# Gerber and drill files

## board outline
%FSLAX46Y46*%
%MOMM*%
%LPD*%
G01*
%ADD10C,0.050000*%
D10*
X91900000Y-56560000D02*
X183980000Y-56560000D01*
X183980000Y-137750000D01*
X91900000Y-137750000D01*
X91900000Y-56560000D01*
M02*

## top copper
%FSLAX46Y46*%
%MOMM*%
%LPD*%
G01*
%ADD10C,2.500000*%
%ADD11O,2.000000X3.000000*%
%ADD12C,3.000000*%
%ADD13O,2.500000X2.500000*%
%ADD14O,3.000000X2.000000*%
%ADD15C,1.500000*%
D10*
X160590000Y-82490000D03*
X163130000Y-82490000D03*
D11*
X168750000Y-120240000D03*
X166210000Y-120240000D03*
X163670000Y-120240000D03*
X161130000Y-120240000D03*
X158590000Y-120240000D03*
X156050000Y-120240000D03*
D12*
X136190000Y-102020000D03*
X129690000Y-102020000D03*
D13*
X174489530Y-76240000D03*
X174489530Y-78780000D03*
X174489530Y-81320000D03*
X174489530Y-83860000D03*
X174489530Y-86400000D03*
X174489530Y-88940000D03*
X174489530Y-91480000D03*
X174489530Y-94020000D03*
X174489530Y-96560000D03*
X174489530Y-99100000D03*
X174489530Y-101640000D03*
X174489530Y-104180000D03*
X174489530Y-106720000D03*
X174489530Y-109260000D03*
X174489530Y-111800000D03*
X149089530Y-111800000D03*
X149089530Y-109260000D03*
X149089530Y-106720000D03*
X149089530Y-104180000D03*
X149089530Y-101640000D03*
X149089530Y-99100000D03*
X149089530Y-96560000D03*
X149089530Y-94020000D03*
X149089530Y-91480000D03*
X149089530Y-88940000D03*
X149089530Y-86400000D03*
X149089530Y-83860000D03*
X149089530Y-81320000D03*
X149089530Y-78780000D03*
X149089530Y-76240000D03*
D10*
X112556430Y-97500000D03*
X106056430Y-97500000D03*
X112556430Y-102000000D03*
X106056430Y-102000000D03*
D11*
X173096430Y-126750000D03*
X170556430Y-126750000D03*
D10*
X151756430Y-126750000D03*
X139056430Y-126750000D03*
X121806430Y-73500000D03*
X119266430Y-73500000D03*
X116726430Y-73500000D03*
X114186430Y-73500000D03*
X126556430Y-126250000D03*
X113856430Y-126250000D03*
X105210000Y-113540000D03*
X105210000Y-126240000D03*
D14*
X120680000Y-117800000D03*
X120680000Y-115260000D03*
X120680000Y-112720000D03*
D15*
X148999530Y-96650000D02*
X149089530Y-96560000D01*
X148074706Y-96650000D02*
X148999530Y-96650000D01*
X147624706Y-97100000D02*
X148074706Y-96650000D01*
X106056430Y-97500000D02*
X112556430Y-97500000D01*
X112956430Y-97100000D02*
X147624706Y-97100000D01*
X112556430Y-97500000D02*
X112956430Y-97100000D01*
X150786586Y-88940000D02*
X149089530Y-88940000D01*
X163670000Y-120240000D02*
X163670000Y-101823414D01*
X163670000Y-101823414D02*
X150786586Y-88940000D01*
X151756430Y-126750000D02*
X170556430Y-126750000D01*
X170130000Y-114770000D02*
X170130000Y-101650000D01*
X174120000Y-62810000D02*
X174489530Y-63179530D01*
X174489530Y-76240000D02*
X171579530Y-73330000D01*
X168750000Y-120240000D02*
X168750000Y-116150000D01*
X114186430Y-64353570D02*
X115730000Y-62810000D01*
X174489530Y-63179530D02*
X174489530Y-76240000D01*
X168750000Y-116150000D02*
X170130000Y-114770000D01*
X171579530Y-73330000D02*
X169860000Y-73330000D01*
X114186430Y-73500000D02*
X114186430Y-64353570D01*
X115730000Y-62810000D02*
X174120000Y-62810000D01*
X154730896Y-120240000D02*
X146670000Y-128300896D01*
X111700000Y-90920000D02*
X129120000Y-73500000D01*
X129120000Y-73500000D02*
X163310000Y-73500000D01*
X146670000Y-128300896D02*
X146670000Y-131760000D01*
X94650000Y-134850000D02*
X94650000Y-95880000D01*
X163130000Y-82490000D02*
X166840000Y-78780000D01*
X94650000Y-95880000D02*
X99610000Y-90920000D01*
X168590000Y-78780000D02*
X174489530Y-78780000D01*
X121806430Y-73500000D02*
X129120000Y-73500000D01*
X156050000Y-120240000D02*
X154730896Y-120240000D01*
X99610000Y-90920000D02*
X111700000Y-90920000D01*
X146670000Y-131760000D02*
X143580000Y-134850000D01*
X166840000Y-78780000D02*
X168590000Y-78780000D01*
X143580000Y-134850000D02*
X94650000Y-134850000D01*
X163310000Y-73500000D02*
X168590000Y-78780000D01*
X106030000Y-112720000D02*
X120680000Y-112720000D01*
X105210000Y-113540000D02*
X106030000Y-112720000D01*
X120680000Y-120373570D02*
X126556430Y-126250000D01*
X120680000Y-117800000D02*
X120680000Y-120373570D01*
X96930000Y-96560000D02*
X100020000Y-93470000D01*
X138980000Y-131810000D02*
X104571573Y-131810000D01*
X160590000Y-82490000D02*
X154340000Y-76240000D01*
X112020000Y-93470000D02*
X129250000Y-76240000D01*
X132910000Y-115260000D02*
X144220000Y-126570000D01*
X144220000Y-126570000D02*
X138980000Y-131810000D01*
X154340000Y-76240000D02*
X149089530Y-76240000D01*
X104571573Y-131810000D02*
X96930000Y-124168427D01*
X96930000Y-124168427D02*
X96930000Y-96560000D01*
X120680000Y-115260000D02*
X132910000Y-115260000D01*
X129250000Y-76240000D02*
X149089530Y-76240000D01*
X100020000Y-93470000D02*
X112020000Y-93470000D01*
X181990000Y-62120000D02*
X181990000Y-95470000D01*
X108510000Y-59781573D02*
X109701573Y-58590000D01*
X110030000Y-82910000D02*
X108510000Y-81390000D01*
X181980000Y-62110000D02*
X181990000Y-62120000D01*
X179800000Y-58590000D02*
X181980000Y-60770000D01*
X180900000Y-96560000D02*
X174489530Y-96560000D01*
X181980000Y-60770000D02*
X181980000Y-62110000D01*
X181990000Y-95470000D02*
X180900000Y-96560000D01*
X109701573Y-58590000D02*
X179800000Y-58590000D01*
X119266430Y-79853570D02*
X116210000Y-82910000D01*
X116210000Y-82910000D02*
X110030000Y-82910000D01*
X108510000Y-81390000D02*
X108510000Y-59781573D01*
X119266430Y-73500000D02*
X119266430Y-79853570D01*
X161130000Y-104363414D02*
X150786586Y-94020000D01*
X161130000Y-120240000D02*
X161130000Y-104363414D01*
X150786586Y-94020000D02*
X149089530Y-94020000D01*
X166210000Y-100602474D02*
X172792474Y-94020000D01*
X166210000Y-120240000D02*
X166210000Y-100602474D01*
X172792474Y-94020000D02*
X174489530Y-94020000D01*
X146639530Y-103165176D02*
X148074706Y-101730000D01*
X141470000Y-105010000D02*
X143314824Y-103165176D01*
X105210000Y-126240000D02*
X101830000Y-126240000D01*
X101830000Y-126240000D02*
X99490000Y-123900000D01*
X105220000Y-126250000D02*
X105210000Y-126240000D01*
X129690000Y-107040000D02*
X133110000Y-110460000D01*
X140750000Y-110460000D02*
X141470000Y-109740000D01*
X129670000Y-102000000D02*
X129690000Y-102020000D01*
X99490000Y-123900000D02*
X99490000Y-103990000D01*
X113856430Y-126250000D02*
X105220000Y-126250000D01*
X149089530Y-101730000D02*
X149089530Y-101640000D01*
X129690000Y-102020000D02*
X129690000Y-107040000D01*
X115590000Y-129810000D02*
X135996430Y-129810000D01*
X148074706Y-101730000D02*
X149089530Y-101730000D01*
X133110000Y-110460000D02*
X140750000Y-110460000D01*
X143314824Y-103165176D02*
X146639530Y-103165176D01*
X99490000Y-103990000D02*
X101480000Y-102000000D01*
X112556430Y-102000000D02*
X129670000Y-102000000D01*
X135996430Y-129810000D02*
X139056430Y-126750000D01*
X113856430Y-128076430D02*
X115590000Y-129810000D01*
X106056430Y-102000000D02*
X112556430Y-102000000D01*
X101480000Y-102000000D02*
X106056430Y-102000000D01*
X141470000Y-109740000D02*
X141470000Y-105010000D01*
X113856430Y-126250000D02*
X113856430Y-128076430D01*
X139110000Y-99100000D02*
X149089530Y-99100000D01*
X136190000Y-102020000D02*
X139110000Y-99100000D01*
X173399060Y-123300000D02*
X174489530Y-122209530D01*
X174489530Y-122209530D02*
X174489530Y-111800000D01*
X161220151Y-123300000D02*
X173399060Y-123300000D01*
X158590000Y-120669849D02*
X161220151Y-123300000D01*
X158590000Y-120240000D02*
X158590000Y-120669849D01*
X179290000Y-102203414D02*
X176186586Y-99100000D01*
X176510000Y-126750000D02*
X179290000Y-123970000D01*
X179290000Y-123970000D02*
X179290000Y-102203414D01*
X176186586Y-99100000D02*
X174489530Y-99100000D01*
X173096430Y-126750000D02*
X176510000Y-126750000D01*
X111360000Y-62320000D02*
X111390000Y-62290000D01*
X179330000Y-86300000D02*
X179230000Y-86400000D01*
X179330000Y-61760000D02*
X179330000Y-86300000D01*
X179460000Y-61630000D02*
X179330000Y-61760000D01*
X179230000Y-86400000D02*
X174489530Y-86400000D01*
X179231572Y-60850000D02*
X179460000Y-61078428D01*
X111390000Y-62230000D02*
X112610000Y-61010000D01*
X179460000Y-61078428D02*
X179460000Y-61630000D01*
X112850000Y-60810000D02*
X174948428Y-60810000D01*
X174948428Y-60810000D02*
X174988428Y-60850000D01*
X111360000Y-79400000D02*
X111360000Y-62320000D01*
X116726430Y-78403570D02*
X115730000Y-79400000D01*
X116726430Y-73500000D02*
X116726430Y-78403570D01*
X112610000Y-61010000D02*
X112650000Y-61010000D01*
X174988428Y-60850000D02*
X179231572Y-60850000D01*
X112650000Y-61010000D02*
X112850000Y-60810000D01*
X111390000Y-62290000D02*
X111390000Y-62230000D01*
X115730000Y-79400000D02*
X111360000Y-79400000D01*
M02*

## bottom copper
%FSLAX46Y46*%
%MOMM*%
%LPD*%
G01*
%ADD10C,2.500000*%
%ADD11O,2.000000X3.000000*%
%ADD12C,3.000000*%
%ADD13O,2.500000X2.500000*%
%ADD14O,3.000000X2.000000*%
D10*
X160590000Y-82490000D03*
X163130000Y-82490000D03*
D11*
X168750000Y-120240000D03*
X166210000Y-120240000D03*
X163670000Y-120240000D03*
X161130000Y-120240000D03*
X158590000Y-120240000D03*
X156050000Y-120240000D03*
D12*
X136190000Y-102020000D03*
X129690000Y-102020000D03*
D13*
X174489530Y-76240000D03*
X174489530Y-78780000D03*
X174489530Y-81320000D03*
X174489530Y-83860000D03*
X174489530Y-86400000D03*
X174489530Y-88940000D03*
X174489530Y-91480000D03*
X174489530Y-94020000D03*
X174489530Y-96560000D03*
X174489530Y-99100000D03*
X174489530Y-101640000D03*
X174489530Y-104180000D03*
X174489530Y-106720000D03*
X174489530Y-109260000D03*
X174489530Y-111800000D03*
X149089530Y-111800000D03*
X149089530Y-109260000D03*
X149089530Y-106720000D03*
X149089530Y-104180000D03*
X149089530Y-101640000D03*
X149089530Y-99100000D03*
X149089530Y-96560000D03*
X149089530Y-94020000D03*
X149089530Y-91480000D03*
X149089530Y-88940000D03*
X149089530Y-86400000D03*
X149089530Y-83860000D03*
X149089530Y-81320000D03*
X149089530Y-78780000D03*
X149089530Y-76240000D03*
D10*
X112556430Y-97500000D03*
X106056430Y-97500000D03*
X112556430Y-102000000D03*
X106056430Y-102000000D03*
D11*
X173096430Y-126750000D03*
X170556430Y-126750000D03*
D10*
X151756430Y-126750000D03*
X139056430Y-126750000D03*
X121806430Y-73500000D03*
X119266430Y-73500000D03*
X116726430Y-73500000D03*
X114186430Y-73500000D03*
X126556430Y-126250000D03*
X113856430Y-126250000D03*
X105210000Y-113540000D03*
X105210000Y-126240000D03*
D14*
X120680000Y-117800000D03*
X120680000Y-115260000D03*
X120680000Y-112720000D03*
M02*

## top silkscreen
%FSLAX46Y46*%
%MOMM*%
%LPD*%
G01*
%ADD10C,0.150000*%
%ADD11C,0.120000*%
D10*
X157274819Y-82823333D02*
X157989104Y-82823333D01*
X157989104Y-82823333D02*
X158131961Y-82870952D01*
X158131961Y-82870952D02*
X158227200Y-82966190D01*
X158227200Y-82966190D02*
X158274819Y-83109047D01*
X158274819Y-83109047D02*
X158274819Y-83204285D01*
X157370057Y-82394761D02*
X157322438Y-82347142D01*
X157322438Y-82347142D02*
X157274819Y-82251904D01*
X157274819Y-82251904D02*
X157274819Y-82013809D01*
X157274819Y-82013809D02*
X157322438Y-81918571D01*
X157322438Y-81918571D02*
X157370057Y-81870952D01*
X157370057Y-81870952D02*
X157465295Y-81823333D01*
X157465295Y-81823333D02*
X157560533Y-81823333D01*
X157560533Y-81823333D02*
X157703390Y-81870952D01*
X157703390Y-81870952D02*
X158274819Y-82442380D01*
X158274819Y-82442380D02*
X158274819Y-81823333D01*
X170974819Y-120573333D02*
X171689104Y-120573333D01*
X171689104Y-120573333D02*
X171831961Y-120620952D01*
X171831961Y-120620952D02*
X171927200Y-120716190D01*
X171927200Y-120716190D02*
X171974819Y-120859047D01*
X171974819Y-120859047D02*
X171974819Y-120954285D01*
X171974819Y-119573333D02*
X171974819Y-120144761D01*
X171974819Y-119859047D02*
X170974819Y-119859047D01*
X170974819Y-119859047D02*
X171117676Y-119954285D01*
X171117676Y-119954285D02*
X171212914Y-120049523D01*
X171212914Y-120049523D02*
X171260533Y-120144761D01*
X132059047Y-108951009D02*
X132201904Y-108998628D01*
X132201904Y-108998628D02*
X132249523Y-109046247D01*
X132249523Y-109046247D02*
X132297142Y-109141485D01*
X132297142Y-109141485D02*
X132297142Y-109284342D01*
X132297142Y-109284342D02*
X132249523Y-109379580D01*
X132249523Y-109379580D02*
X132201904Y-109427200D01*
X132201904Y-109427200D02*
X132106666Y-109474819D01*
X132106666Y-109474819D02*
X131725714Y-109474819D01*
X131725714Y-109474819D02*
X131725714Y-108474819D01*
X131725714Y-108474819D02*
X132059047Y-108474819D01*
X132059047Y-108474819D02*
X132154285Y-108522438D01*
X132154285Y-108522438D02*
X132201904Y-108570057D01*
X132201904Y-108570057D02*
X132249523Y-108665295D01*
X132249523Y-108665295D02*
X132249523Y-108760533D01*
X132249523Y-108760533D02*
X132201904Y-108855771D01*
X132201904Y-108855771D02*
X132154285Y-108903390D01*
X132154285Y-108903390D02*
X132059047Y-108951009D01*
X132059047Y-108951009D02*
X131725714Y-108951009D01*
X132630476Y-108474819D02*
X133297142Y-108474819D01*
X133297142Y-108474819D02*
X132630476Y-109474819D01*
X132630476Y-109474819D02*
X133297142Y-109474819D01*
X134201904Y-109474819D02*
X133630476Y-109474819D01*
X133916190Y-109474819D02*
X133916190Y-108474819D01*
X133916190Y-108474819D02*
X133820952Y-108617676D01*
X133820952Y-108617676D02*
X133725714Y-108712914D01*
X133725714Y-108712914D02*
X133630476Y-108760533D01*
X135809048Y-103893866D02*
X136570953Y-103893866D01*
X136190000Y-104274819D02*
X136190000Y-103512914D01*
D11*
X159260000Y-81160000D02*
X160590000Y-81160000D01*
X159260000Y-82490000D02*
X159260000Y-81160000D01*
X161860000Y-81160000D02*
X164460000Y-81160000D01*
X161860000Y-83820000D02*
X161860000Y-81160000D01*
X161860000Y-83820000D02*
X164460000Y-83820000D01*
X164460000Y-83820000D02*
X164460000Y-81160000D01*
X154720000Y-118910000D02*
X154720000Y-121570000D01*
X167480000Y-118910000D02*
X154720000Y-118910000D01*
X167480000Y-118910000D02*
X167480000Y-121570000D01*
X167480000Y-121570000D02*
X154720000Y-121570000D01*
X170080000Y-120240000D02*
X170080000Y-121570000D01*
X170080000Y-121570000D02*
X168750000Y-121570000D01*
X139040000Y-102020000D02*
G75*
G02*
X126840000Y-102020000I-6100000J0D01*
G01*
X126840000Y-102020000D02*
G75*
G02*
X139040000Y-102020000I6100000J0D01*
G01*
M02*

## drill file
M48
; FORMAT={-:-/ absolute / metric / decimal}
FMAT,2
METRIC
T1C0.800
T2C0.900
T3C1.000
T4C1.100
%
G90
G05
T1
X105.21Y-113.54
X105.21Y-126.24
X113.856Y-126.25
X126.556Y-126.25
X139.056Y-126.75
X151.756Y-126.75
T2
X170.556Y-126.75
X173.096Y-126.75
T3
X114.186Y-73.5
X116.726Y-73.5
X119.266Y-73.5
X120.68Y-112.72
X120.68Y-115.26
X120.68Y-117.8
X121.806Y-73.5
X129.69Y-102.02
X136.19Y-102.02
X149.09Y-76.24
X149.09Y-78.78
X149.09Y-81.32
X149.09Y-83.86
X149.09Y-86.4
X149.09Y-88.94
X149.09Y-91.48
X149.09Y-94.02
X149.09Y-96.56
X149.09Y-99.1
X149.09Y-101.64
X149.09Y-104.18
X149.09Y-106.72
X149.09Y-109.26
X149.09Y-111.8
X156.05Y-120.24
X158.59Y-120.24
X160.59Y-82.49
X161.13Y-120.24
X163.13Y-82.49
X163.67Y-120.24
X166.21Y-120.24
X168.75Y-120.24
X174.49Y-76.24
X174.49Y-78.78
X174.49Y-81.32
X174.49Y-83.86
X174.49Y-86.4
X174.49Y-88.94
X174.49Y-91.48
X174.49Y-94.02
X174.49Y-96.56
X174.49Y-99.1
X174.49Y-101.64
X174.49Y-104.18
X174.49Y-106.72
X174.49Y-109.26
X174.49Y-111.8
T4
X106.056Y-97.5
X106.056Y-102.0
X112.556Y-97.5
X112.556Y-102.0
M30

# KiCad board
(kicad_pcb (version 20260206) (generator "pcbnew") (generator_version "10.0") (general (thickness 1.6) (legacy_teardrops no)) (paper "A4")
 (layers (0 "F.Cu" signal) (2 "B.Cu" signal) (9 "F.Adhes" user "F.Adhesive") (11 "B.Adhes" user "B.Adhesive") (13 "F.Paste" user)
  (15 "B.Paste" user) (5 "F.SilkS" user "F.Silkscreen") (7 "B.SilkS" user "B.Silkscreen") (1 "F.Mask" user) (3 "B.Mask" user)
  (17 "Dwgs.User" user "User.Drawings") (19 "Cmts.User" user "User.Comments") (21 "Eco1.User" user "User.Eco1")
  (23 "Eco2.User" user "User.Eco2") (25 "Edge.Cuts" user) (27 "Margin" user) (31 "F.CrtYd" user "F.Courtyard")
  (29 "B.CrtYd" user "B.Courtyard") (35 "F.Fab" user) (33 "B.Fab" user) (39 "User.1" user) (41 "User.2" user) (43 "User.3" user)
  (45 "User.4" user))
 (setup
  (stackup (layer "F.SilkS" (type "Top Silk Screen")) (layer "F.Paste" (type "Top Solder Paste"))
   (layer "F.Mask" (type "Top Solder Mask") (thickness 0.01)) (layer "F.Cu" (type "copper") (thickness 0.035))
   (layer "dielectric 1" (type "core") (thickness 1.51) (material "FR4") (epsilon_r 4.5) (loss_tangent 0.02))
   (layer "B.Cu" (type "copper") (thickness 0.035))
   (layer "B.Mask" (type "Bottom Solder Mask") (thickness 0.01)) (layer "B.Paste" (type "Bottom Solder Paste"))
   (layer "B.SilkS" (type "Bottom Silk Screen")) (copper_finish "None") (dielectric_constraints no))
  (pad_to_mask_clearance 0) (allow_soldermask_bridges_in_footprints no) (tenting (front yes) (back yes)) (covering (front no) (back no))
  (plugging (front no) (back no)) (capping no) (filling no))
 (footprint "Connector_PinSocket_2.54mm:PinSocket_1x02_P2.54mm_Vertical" (layer "F.Cu") (at 160.59 82.49 90)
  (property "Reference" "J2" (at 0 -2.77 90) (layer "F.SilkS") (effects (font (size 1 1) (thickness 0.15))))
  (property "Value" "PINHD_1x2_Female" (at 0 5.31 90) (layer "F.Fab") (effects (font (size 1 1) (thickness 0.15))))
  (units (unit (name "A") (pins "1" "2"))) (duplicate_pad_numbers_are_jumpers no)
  (fp_line (start 1.33 -1.33) (end 1.33 0) (stroke (width 0.12) (type solid)) (layer "F.SilkS"))
  (fp_line (start 0 -1.33) (end 1.33 -1.33) (stroke (width 0.12) (type solid)) (layer "F.SilkS"))
  (fp_line (start 1.33 1.27) (end 1.33 3.87) (stroke (width 0.12) (type solid)) (layer "F.SilkS"))
  (fp_line (start -1.33 1.27) (end 1.33 1.27) (stroke (width 0.12) (type solid)) (layer "F.SilkS"))
  (fp_line (start -1.33 1.27) (end -1.33 3.87) (stroke (width 0.12) (type solid)) (layer "F.SilkS"))
  (fp_line (start -1.33 3.87) (end 1.33 3.87) (stroke (width 0.12) (type solid)) (layer "F.SilkS"))
  (pad "1" thru_hole circle (at 0 0 90) (size 2.5 2.5) (drill 1) (layers "*.Cu" "*.Mask") (remove_unused_layers no) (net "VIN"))
  (pad "2" thru_hole circle (at 0 2.54 90) (size 2.5 2.5) (drill 1) (layers "*.Cu" "*.Mask") (remove_unused_layers no) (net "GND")))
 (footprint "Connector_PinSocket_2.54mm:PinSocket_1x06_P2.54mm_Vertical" (layer "F.Cu") (at 168.75 120.24 -90)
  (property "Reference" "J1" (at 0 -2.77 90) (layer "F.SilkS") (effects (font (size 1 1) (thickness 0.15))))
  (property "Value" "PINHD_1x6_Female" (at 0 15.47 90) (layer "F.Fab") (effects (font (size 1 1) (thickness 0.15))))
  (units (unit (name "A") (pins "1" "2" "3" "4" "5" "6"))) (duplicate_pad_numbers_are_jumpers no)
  (fp_line (start -1.33 14.03) (end 1.33 14.03) (stroke (width 0.12) (type solid)) (layer "F.SilkS"))
  (fp_line (start -1.33 1.27) (end -1.33 14.03) (stroke (width 0.12) (type solid)) (layer "F.SilkS"))
  (fp_line (start -1.33 1.27) (end 1.33 1.27) (stroke (width 0.12) (type solid)) (layer "F.SilkS"))
  (fp_line (start 1.33 1.27) (end 1.33 14.03) (stroke (width 0.12) (type solid)) (layer "F.SilkS"))
  (fp_line (start 0 -1.33) (end 1.33 -1.33) (stroke (width 0.12) (type solid)) (layer "F.SilkS"))
  (fp_line (start 1.33 -1.33) (end 1.33 0) (stroke (width 0.12) (type solid)) (layer "F.SilkS"))
  (pad "1" thru_hole oval (at 0 0 270) (size 3 2) (drill 1) (layers "*.Cu" "*.Mask") (remove_unused_layers no) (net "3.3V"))
  (pad "2" thru_hole oval (at 0 2.54 270) (size 3 2) (drill 1) (layers "*.Cu" "*.Mask") (remove_unused_layers no) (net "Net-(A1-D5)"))
  (pad "3" thru_hole oval (at 0 5.08 270) (size 3 2) (drill 1) (layers "*.Cu" "*.Mask") (remove_unused_layers no)
   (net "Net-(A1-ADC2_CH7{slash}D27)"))
  (pad "4" thru_hole oval (at 0 7.62 270) (size 3 2) (drill 1) (layers "*.Cu" "*.Mask") (remove_unused_layers no)
   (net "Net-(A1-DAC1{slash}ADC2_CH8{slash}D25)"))
  (pad "5" thru_hole oval (at 0 10.16 270) (size 3 2) (drill 1) (layers "*.Cu" "*.Mask") (remove_unused_layers no) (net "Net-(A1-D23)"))
  (pad "6" thru_hole oval (at 0 12.7 270) (size 3 2) (drill 1) (layers "*.Cu" "*.Mask") (remove_unused_layers no) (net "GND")))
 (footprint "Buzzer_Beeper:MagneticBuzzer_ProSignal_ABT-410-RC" (layer "F.Cu") (at 136.19 102.02 180)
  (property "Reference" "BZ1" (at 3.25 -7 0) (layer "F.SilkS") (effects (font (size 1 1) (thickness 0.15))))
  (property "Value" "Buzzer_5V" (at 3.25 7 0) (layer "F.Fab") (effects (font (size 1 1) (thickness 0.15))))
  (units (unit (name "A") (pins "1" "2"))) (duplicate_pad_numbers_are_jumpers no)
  (fp_circle (center 3.25 0) (end 9.35 0) (stroke (width 0.12) (type solid)) (fill no) (layer "F.SilkS"))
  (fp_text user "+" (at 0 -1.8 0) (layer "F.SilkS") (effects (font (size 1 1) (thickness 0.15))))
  (pad "1" thru_hole circle (at 0 0 180) (size 3 3) (drill 1) (layers "*.Cu" "*.Mask") (remove_unused_layers no)
   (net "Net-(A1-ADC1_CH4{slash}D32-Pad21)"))
  (pad "2" thru_hole circle (at 6.5 0 180) (size 3 3) (drill 1) (layers "*.Cu" "*.Mask") (remove_unused_layers no)
   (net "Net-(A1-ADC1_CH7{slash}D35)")))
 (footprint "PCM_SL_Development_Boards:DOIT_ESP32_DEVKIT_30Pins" (layer "B.Cu") (at 174.48953 76.24 180)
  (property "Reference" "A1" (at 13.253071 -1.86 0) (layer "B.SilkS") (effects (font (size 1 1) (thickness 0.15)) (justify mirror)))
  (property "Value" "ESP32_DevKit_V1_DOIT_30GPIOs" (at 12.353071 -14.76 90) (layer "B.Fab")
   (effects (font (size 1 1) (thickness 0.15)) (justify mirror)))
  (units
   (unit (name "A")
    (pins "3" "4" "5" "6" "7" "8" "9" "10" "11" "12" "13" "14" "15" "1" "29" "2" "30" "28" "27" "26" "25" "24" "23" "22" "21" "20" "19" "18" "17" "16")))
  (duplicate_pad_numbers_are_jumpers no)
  (pad "1" thru_hole oval (at 0 0 90) (size 2.5 2.5) (drill 1) (layers "*.Cu" "*.Mask") (remove_unused_layers no) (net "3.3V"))
  (pad "2" thru_hole oval (at 0 -2.54 90) (size 2.5 2.5) (drill 1) (layers "*.Cu" "*.Mask") (remove_unused_layers no) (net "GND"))
  (pad "3" thru_hole oval (at 0 -5.08 90) (size 2.5 2.5) (drill 1) (layers "*.Cu" "*.Mask") (remove_unused_layers no)
   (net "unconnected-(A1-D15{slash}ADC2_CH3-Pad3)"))
  (pad "4" thru_hole oval (at 0 -7.62 90) (size 2.5 2.5) (drill 1) (layers "*.Cu" "*.Mask") (remove_unused_layers no)
   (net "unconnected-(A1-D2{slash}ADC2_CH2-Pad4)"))
  (pad "5" thru_hole oval (at 0 -10.16 90) (size 2.5 2.5) (drill 1) (layers "*.Cu" "*.Mask") (remove_unused_layers no)
   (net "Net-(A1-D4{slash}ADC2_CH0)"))
  (pad "6" thru_hole oval (at 0 -12.7 90) (size 2.5 2.5) (drill 1) (layers "*.Cu" "*.Mask") (remove_unused_layers no)
   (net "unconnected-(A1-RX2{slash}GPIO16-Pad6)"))
  (pad "7" thru_hole oval (at 0 -15.24 90) (size 2.5 2.5) (drill 1) (layers "*.Cu" "*.Mask") (remove_unused_layers no)
   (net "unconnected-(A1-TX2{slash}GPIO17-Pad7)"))
  (pad "8" thru_hole oval (at 0 -17.78 90) (size 2.5 2.5) (drill 1) (layers "*.Cu" "*.Mask") (remove_unused_layers no) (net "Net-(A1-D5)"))
  (pad "9" thru_hole oval (at 0 -20.32 90) (size 2.5 2.5) (drill 1) (layers "*.Cu" "*.Mask") (remove_unused_layers no) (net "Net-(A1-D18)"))
  (pad "10" thru_hole oval (at 0 -22.86 90) (size 2.5 2.5) (drill 1) (layers "*.Cu" "*.Mask") (remove_unused_layers no) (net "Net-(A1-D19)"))
  (pad "11" thru_hole oval (at 0 -25.4 90) (size 2.5 2.5) (drill 1) (layers "*.Cu" "*.Mask") (remove_unused_layers no)
   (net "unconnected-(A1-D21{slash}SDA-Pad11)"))
  (pad "12" thru_hole oval (at 0 -27.94 90) (size 2.5 2.5) (drill 1) (layers "*.Cu" "*.Mask") (remove_unused_layers no)
   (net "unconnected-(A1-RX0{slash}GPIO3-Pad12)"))
  (pad "13" thru_hole oval (at 0 -30.48 90) (size 2.5 2.5) (drill 1) (layers "*.Cu" "*.Mask") (remove_unused_layers no)
   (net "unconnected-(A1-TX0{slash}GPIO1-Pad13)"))
  (pad "14" thru_hole oval (at 0 -33.02 90) (size 2.5 2.5) (drill 1) (layers "*.Cu" "*.Mask") (remove_unused_layers no)
   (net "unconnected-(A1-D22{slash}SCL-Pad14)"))
  (pad "15" thru_hole oval (at 0 -35.56 90) (size 2.5 2.5) (drill 1) (layers "*.Cu" "*.Mask") (remove_unused_layers no) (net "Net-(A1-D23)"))
  (pad "16" thru_hole oval (at 25.4 -35.56 90) (size 2.5 2.5) (drill 1) (layers "*.Cu" "*.Mask") (remove_unused_layers no)
   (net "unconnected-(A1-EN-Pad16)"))
  (pad "17" thru_hole oval (at 25.4 -33.02 90) (size 2.5 2.5) (drill 1) (layers "*.Cu" "*.Mask") (remove_unused_layers no)
   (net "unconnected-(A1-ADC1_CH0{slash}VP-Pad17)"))
  (pad "18" thru_hole oval (at 25.4 -30.48 90) (size 2.5 2.5) (drill 1) (layers "*.Cu" "*.Mask") (remove_unused_layers no)
   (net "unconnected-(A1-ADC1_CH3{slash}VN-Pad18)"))
  (pad "19" thru_hole oval (at 25.4 -27.94 90) (size 2.5 2.5) (drill 1) (layers "*.Cu" "*.Mask") (remove_unused_layers no)
   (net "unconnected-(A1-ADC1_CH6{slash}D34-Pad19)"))
  (pad "20" thru_hole oval (at 25.4 -25.4 90) (size 2.5 2.5) (drill 1) (layers "*.Cu" "*.Mask") (remove_unused_layers no)
   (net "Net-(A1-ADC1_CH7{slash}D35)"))
  (pad "21" thru_hole oval (at 25.4 -22.86 90) (size 2.5 2.5) (drill 1) (layers "*.Cu" "*.Mask") (remove_unused_layers no)
   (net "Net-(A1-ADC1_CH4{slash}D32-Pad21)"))
  (pad "22" thru_hole oval (at 25.4 -20.32 90) (size 2.5 2.5) (drill 1) (layers "*.Cu" "*.Mask") (remove_unused_layers no)
   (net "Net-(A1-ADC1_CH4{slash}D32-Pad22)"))
  (pad "23" thru_hole oval (at 25.4 -17.78 90) (size 2.5 2.5) (drill 1) (layers "*.Cu" "*.Mask") (remove_unused_layers no)
   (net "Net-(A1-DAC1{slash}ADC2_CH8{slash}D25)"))
  (pad "24" thru_hole oval (at 25.4 -15.24 90) (size 2.5 2.5) (drill 1) (layers "*.Cu" "*.Mask") (remove_unused_layers no)
   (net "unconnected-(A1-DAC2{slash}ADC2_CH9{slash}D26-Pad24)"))
  (pad "25" thru_hole oval (at 25.4 -12.7 90) (size 2.5 2.5) (drill 1) (layers "*.Cu" "*.Mask") (remove_unused_layers no)
   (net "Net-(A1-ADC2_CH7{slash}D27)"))
  (pad "26" thru_hole oval (at 25.4 -10.16 90) (size 2.5 2.5) (drill 1) (layers "*.Cu" "*.Mask") (remove_unused_layers no)
   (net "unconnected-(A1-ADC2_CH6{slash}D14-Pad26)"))
  (pad "27" thru_hole oval (at 25.4 -7.62 90) (size 2.5 2.5) (drill 1) (layers "*.Cu" "*.Mask") (remove_unused_layers no)
   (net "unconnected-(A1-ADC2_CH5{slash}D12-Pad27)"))
  (pad "28" thru_hole oval (at 25.4 -5.08 90) (size 2.5 2.5) (drill 1) (layers "*.Cu" "*.Mask") (remove_unused_layers no)
   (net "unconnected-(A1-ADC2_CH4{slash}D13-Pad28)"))
  (pad "29" thru_hole oval (at 25.4 -2.54 90) (size 2.5 2.5) (drill 1) (layers "*.Cu" "*.Mask") (remove_unused_layers no)
   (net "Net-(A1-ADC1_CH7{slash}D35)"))
  (pad "30" thru_hole oval (at 25.4 0 90) (size 2.5 2.5) (drill 1) (layers "*.Cu" "*.Mask") (remove_unused_layers no) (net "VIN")))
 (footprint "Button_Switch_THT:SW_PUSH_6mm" (layer "B.Cu") (at 112.55643 97.5 180)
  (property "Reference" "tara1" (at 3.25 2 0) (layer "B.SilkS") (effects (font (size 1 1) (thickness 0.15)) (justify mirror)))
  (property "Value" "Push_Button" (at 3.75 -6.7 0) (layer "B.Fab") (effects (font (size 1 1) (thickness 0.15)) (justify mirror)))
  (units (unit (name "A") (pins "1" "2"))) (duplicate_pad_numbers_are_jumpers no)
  (pad "1" thru_hole circle (at 0 0 90) (size 2.5 2.5) (drill 1.1) (layers "*.Cu" "*.Mask") (remove_unused_layers no)
   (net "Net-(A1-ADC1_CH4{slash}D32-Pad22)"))
  (pad "1" thru_hole circle (at 6.5 0 90) (size 2.5 2.5) (drill 1.1) (layers "*.Cu" "*.Mask") (remove_unused_layers no)
   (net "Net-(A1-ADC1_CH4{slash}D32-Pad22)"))
  (pad "2" thru_hole circle (at 0 -4.5 90) (size 2.5 2.5) (drill 1.1) (layers "*.Cu" "*.Mask") (remove_unused_layers no)
   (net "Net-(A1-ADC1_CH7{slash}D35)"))
  (pad "2" thru_hole circle (at 6.5 -4.5 90) (size 2.5 2.5) (drill 1.1) (layers "*.Cu" "*.Mask") (remove_unused_layers no)
   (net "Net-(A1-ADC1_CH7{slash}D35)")))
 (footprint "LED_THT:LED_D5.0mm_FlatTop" (layer "B.Cu") (at 173.09643 126.75 180)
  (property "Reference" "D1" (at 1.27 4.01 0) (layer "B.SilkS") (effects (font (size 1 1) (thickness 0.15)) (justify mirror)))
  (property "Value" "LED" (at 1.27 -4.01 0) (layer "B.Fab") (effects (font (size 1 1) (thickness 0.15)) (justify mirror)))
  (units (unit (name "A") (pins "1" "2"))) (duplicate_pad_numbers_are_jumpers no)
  (pad "1" thru_hole oval (at 0 0 180) (size 2 3) (drill 0.9) (layers "*.Cu" "*.Mask") (remove_unused_layers no) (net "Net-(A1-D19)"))
  (pad "2" thru_hole oval (at 2.54 0 180) (size 2 3) (drill 0.9) (layers "*.Cu" "*.Mask") (remove_unused_layers no) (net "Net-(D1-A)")))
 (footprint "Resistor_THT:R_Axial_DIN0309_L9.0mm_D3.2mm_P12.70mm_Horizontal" (layer "B.Cu") (at 151.75643 126.75 180)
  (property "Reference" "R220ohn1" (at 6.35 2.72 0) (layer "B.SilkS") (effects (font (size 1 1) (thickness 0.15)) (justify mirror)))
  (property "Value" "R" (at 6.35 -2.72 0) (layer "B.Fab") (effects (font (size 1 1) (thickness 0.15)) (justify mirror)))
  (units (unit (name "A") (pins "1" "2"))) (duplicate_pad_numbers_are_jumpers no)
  (pad "1" thru_hole circle (at 0 0 180) (size 2.5 2.5) (drill 0.8) (layers "*.Cu" "*.Mask") (remove_unused_layers no) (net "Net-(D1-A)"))
  (pad "2" thru_hole circle (at 12.7 0 180) (size 2.5 2.5) (drill 0.8) (layers "*.Cu" "*.Mask") (remove_unused_layers no)
   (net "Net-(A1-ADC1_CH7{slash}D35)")))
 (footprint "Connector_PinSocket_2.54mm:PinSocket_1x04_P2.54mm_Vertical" (layer "B.Cu") (at 121.80643 73.5 90)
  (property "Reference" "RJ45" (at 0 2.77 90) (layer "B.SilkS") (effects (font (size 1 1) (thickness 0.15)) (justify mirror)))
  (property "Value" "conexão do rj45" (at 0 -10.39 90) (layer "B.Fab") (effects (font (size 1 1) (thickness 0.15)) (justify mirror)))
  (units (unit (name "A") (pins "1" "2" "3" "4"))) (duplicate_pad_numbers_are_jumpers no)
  (pad "1" thru_hole circle (at 0 0 90) (size 2.5 2.5) (drill 1) (layers "*.Cu" "*.Mask") (remove_unused_layers no) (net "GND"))
  (pad "2" thru_hole circle (at 0 -2.54 90) (size 2.5 2.5) (drill 1) (layers "*.Cu" "*.Mask") (remove_unused_layers no) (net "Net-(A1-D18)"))
  (pad "3" thru_hole circle (at 0 -5.08 90) (size 2.5 2.5) (drill 1) (layers "*.Cu" "*.Mask") (remove_unused_layers no)
   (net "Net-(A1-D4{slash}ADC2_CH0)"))
  (pad "4" thru_hole circle (at 0 -7.62 90) (size 2.5 2.5) (drill 1) (layers "*.Cu" "*.Mask") (remove_unused_layers no) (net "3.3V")))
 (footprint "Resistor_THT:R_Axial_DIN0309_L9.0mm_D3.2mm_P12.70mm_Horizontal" (layer "B.Cu") (at 126.55643 126.25 180)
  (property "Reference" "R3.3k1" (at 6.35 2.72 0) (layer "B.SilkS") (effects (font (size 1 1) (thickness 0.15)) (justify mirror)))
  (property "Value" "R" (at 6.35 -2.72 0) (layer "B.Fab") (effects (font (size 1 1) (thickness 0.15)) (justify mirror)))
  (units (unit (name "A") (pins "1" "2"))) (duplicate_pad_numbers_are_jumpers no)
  (pad "1" thru_hole circle (at 0 0 180) (size 2.5 2.5) (drill 0.8) (layers "*.Cu" "*.Mask") (remove_unused_layers no)
   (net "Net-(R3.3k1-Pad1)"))
  (pad "2" thru_hole circle (at 12.7 0 180) (size 2.5 2.5) (drill 0.8) (layers "*.Cu" "*.Mask") (remove_unused_layers no)
   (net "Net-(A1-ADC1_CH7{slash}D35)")))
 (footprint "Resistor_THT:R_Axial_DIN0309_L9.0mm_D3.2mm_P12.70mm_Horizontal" (layer "B.Cu") (at 105.21 113.54 -90)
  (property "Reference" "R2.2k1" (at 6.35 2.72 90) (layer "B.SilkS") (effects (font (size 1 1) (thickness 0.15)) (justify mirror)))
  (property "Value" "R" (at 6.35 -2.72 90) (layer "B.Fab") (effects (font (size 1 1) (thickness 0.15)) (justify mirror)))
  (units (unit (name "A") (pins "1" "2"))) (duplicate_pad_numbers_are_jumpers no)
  (pad "1" thru_hole circle (at 0 0 270) (size 2.5 2.5) (drill 0.8) (layers "*.Cu" "*.Mask") (remove_unused_layers no)
   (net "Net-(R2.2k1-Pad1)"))
  (pad "2" thru_hole circle (at 12.7 0 270) (size 2.5 2.5) (drill 0.8) (layers "*.Cu" "*.Mask") (remove_unused_layers no)
   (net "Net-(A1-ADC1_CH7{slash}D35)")))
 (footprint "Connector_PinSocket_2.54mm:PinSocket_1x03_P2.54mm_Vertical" (layer "B.Cu") (at 120.68 117.8)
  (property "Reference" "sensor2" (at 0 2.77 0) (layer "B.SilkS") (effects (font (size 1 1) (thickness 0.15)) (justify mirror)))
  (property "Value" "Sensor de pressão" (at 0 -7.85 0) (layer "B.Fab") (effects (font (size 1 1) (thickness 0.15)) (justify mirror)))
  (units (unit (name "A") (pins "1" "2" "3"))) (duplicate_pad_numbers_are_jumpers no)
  (pad "1" thru_hole oval (at 0 0) (size 3 2) (drill 1) (layers "*.Cu" "*.Mask") (remove_unused_layers no) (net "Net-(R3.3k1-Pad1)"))
  (pad "2" thru_hole oval (at 0 -2.54) (size 3 2) (drill 1) (layers "*.Cu" "*.Mask") (remove_unused_layers no) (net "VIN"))
  (pad "3" thru_hole oval (at 0 -5.08) (size 3 2) (drill 1) (layers "*.Cu" "*.Mask") (remove_unused_layers no) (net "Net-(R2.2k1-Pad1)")))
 (gr_rect (start 91.9 56.56) (end 183.98 137.75) (stroke (width 0.05) (type default)) (fill no) (layer "Edge.Cuts"))
 (segment (start 148.99953 96.65) (end 149.08953 96.56) (width 1.5) (layer "F.Cu") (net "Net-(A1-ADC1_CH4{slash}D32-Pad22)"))
 (segment (start 148.074706 96.65) (end 148.99953 96.65) (width 1.5) (layer "F.Cu") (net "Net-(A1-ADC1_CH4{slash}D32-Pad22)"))
 (segment (start 147.624706 97.1) (end 148.074706 96.65) (width 1.5) (layer "F.Cu") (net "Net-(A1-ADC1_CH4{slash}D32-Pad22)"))
 (segment (start 106.05643 97.5) (end 112.55643 97.5) (width 1.5) (layer "F.Cu") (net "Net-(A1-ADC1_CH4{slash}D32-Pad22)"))
 (segment (start 112.95643 97.1) (end 147.624706 97.1) (width 1.5) (layer "F.Cu") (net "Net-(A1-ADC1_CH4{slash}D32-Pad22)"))
 (segment (start 112.55643 97.5) (end 112.95643 97.1) (width 1.5) (layer "F.Cu") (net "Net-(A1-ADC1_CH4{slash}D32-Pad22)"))
 (segment (start 150.786586 88.94) (end 149.08953 88.94) (width 1.5) (layer "F.Cu") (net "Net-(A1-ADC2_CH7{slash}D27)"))
 (segment (start 163.67 120.24) (end 163.67 101.823414) (width 1.5) (layer "F.Cu") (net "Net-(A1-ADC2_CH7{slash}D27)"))
 (segment (start 163.67 101.823414) (end 150.786586 88.94) (width 1.5) (layer "F.Cu") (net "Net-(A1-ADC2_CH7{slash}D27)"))
 (segment (start 151.75643 126.75) (end 170.55643 126.75) (width 1.5) (layer "F.Cu") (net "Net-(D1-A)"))
 (segment (start 170.13 114.77) (end 170.13 101.65) (width 1.5) (layer "F.Cu") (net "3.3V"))
 (segment (start 174.12 62.81) (end 174.48953 63.17953) (width 1.5) (layer "F.Cu") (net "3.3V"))
 (segment (start 174.48953 76.24) (end 171.57953 73.33) (width 1.5) (layer "F.Cu") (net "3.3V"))
 (segment (start 168.75 120.24) (end 168.75 116.15) (width 1.5) (layer "F.Cu") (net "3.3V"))
 (segment (start 114.18643 64.35357) (end 115.73 62.81) (width 1.5) (layer "F.Cu") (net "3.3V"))
 (segment (start 174.48953 63.17953) (end 174.48953 76.24) (width 1.5) (layer "F.Cu") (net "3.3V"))
 (segment (start 168.75 116.15) (end 170.13 114.77) (width 1.5) (layer "F.Cu") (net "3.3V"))
 (segment (start 171.57953 73.33) (end 169.86 73.33) (width 1.5) (layer "F.Cu") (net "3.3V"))
 (segment (start 114.18643 73.5) (end 114.18643 64.35357) (width 1.5) (layer "F.Cu") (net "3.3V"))
 (segment (start 115.73 62.81) (end 174.12 62.81) (width 1.5) (layer "F.Cu") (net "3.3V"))
 (segment (start 154.730896 120.24) (end 146.67 128.300896) (width 1.5) (layer "F.Cu") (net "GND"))
 (segment (start 111.7 90.92) (end 129.12 73.5) (width 1.5) (layer "F.Cu") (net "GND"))
 (segment (start 129.12 73.5) (end 163.31 73.5) (width 1.5) (layer "F.Cu") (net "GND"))
 (segment (start 146.67 128.300896) (end 146.67 131.76) (width 1.5) (layer "F.Cu") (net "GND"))
 (segment (start 94.65 134.85) (end 94.65 95.88) (width 1.5) (layer "F.Cu") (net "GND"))
 (segment (start 163.13 82.49) (end 166.84 78.78) (width 1.5) (layer "F.Cu") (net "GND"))
 (segment (start 94.65 95.88) (end 99.61 90.92) (width 1.5) (layer "F.Cu") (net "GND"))
 (segment (start 168.59 78.78) (end 174.48953 78.78) (width 1.5) (layer "F.Cu") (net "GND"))
 (segment (start 121.80643 73.5) (end 129.12 73.5) (width 1.5) (layer "F.Cu") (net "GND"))
 (segment (start 156.05 120.24) (end 154.730896 120.24) (width 1.5) (layer "F.Cu") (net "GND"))
 (segment (start 99.61 90.92) (end 111.7 90.92) (width 1.5) (layer "F.Cu") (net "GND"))
 (segment (start 146.67 131.76) (end 143.58 134.85) (width 1.5) (layer "F.Cu") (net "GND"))
 (segment (start 166.84 78.78) (end 168.59 78.78) (width 1.5) (layer "F.Cu") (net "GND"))
 (segment (start 143.58 134.85) (end 94.65 134.85) (width 1.5) (layer "F.Cu") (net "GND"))
 (segment (start 163.31 73.5) (end 168.59 78.78) (width 1.5) (layer "F.Cu") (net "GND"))
 (segment (start 106.03 112.72) (end 120.68 112.72) (width 1.5) (layer "F.Cu") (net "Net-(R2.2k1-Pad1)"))
 (segment (start 105.21 113.54) (end 106.03 112.72) (width 1.5) (layer "F.Cu") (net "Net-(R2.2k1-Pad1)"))
 (segment (start 120.68 120.37357) (end 126.55643 126.25) (width 1.5) (layer "F.Cu") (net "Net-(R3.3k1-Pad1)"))
 (segment (start 120.68 117.8) (end 120.68 120.37357) (width 1.5) (layer "F.Cu") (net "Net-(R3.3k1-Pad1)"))
 (segment (start 96.93 96.56) (end 100.02 93.47) (width 1.5) (layer "F.Cu") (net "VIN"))
 (segment (start 138.98 131.81) (end 104.571573 131.81) (width 1.5) (layer "F.Cu") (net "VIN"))
 (segment (start 160.59 82.49) (end 154.34 76.24) (width 1.5) (layer "F.Cu") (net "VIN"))
 (segment (start 112.02 93.47) (end 129.25 76.24) (width 1.5) (layer "F.Cu") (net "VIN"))
 (segment (start 132.91 115.26) (end 144.22 126.57) (width 1.5) (layer "F.Cu") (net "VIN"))
 (segment (start 144.22 126.57) (end 138.98 131.81) (width 1.5) (layer "F.Cu") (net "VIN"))
 (segment (start 154.34 76.24) (end 149.08953 76.24) (width 1.5) (layer "F.Cu") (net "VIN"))
 (segment (start 104.571573 131.81) (end 96.93 124.168427) (width 1.5) (layer "F.Cu") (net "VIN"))
 (segment (start 96.93 124.168427) (end 96.93 96.56) (width 1.5) (layer "F.Cu") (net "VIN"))
 (segment (start 120.68 115.26) (end 132.91 115.26) (width 1.5) (layer "F.Cu") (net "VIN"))
 (segment (start 129.25 76.24) (end 149.08953 76.24) (width 1.5) (layer "F.Cu") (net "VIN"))
 (segment (start 100.02 93.47) (end 112.02 93.47) (width 1.5) (layer "F.Cu") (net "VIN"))
 (segment (start 181.99 62.12) (end 181.99 95.47) (width 1.5) (layer "F.Cu") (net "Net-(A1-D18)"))
 (segment (start 108.51 59.781573) (end 109.701573 58.59) (width 1.5) (layer "F.Cu") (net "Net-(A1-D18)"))
 (segment (start 110.03 82.91) (end 108.51 81.39) (width 1.5) (layer "F.Cu") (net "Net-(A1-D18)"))
 (segment (start 181.98 62.11) (end 181.99 62.12) (width 1.5) (layer "F.Cu") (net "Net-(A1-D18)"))
 (segment (start 179.8 58.59) (end 181.98 60.77) (width 1.5) (layer "F.Cu") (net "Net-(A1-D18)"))
 (segment (start 180.9 96.56) (end 174.48953 96.56) (width 1.5) (layer "F.Cu") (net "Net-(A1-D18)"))
 (segment (start 181.98 60.77) (end 181.98 62.11) (width 1.5) (layer "F.Cu") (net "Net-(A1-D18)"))
 (segment (start 181.99 95.47) (end 180.9 96.56) (width 1.5) (layer "F.Cu") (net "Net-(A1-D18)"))
 (segment (start 109.701573 58.59) (end 179.8 58.59) (width 1.5) (layer "F.Cu") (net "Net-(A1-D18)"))
 (segment (start 119.26643 79.85357) (end 116.21 82.91) (width 1.5) (layer "F.Cu") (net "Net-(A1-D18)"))
 (segment (start 116.21 82.91) (end 110.03 82.91) (width 1.5) (layer "F.Cu") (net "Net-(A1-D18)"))
 (segment (start 108.51 81.39) (end 108.51 59.781573) (width 1.5) (layer "F.Cu") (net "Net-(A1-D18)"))
 (segment (start 119.26643 73.5) (end 119.26643 79.85357) (width 1.5) (layer "F.Cu") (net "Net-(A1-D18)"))
 (segment (start 161.13 104.363414) (end 150.786586 94.02) (width 1.5) (layer "F.Cu") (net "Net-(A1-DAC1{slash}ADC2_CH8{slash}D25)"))
 (segment (start 161.13 120.24) (end 161.13 104.363414) (width 1.5) (layer "F.Cu") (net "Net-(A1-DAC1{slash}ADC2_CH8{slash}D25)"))
 (segment (start 150.786586 94.02) (end 149.08953 94.02) (width 1.5) (layer "F.Cu") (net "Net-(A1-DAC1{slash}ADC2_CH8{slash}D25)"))
 (segment (start 166.21 100.602474) (end 172.792474 94.02) (width 1.5) (layer "F.Cu") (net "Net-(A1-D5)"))
 (segment (start 166.21 120.24) (end 166.21 100.602474) (width 1.5) (layer "F.Cu") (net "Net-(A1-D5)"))
 (segment (start 172.792474 94.02) (end 174.48953 94.02) (width 1.5) (layer "F.Cu") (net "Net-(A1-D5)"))
 (segment (start 146.63953 103.165176) (end 148.074706 101.73) (width 1.5) (layer "F.Cu") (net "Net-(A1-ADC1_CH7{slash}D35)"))
 (segment (start 141.47 105.01) (end 143.314824 103.165176) (width 1.5) (layer "F.Cu") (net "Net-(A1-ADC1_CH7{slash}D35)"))
 (segment (start 105.21 126.24) (end 101.83 126.24) (width 1.5) (layer "F.Cu") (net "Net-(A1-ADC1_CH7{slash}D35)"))
 (segment (start 101.83 126.24) (end 99.49 123.9) (width 1.5) (layer "F.Cu") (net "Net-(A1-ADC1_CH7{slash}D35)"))
 (segment (start 105.22 126.25) (end 105.21 126.24) (width 1.5) (layer "F.Cu") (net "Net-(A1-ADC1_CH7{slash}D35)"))
 (segment (start 129.69 107.04) (end 133.11 110.46) (width 1.5) (layer "F.Cu") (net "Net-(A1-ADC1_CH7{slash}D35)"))
 (segment (start 140.75 110.46) (end 141.47 109.74) (width 1.5) (layer "F.Cu") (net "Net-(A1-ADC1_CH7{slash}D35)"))
 (segment (start 129.67 102) (end 129.69 102.02) (width 1.5) (layer "F.Cu") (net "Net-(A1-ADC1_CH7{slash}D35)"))
 (segment (start 99.49 123.9) (end 99.49 103.99) (width 1.5) (layer "F.Cu") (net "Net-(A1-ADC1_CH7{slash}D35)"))
 (segment (start 113.85643 126.25) (end 105.22 126.25) (width 1.5) (layer "F.Cu") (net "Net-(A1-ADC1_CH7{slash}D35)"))
 (segment (start 149.08953 101.73) (end 149.08953 101.64) (width 1.5) (layer "F.Cu") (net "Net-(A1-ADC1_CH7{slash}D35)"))
 (segment (start 129.69 102.02) (end 129.69 107.04) (width 1.5) (layer "F.Cu") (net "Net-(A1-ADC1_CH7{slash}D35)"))
 (segment (start 115.59 129.81) (end 135.99643 129.81) (width 1.5) (layer "F.Cu") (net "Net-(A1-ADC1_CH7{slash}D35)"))
 (segment (start 148.074706 101.73) (end 149.08953 101.73) (width 1.5) (layer "F.Cu") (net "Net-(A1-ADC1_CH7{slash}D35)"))
 (segment (start 133.11 110.46) (end 140.75 110.46) (width 1.5) (layer "F.Cu") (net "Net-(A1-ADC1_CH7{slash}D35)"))
 (segment (start 143.314824 103.165176) (end 146.63953 103.165176) (width 1.5) (layer "F.Cu") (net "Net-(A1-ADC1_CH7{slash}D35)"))
 (segment (start 99.49 103.99) (end 101.48 102) (width 1.5) (layer "F.Cu") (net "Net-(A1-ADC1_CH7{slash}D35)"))
 (segment (start 112.55643 102) (end 129.67 102) (width 1.5) (layer "F.Cu") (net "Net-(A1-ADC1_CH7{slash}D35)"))
 (segment (start 135.99643 129.81) (end 139.05643 126.75) (width 1.5) (layer "F.Cu") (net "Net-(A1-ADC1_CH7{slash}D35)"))
 (segment (start 113.85643 128.07643) (end 115.59 129.81) (width 1.5) (layer "F.Cu") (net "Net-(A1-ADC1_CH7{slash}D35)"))
 (segment (start 106.05643 102) (end 112.55643 102) (width 1.5) (layer "F.Cu") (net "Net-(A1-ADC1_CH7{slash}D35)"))
 (segment (start 101.48 102) (end 106.05643 102) (width 1.5) (layer "F.Cu") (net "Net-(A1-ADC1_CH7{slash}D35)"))
 (segment (start 141.47 109.74) (end 141.47 105.01) (width 1.5) (layer "F.Cu") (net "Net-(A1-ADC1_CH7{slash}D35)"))
 (segment (start 113.85643 126.25) (end 113.85643 128.07643) (width 1.5) (layer "F.Cu") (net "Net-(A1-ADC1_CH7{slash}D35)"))
 (segment (start 139.11 99.1) (end 149.08953 99.1) (width 1.5) (layer "F.Cu") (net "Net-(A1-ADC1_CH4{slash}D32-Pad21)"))
 (segment (start 136.19 102.02) (end 139.11 99.1) (width 1.5) (layer "F.Cu") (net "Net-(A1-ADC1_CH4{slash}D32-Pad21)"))
 (segment (start 173.39906 123.3) (end 174.48953 122.20953) (width 1.5) (layer "F.Cu") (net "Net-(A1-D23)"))
 (segment (start 174.48953 122.20953) (end 174.48953 111.8) (width 1.5) (layer "F.Cu") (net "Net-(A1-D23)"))
 (segment (start 161.220151 123.3) (end 173.39906 123.3) (width 1.5) (layer "F.Cu") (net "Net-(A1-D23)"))
 (segment (start 158.59 120.669849) (end 161.220151 123.3) (width 1.5) (layer "F.Cu") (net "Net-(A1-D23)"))
 (segment (start 158.59 120.24) (end 158.59 120.669849) (width 1.5) (layer "F.Cu") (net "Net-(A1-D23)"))
 (segment (start 179.29 102.203414) (end 176.186586 99.1) (width 1.5) (layer "F.Cu") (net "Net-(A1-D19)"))
 (segment (start 176.51 126.75) (end 179.29 123.97) (width 1.5) (layer "F.Cu") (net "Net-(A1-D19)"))
 (segment (start 179.29 123.97) (end 179.29 102.203414) (width 1.5) (layer "F.Cu") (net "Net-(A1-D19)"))
 (segment (start 176.186586 99.1) (end 174.48953 99.1) (width 1.5) (layer "F.Cu") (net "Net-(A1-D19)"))
 (segment (start 173.09643 126.75) (end 176.51 126.75) (width 1.5) (layer "F.Cu") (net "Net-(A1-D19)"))
 (segment (start 111.36 62.32) (end 111.39 62.29) (width 1.5) (layer "F.Cu") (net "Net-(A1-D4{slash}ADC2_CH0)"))
 (segment (start 179.33 86.3) (end 179.23 86.4) (width 1.5) (layer "F.Cu") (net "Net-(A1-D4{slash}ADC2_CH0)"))
 (segment (start 179.33 61.76) (end 179.33 86.3) (width 1.5) (layer "F.Cu") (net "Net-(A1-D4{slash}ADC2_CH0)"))
 (segment (start 179.46 61.63) (end 179.33 61.76) (width 1.5) (layer "F.Cu") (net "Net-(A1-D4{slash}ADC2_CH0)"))
 (segment (start 179.23 86.4) (end 174.48953 86.4) (width 1.5) (layer "F.Cu") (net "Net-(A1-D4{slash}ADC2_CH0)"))
 (segment (start 179.231572 60.85) (end 179.46 61.078428) (width 1.5) (layer "F.Cu") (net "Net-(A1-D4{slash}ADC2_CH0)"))
 (segment (start 111.39 62.23) (end 112.61 61.01) (width 1.5) (layer "F.Cu") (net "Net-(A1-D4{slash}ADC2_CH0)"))
 (segment (start 179.46 61.078428) (end 179.46 61.63) (width 1.5) (layer "F.Cu") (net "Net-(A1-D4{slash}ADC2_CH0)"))
 (segment (start 112.85 60.81) (end 174.948428 60.81) (width 1.5) (layer "F.Cu") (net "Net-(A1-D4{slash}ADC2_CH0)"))
 (segment (start 174.948428 60.81) (end 174.988428 60.85) (width 1.5) (layer "F.Cu") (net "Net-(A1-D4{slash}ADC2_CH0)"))
 (segment (start 111.36 79.4) (end 111.36 62.32) (width 1.5) (layer "F.Cu") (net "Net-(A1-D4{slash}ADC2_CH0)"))
 (segment (start 116.72643 78.40357) (end 115.73 79.4) (width 1.5) (layer "F.Cu") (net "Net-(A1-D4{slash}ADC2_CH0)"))
 (segment (start 116.72643 73.5) (end 116.72643 78.40357) (width 1.5) (layer "F.Cu") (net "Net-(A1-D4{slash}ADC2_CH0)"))
 (segment (start 112.61 61.01) (end 112.65 61.01) (width 1.5) (layer "F.Cu") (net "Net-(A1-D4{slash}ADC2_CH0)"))
 (segment (start 174.988428 60.85) (end 179.231572 60.85) (width 1.5) (layer "F.Cu") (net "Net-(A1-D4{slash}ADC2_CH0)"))
 (segment (start 112.65 61.01) (end 112.85 60.81) (width 1.5) (layer "F.Cu") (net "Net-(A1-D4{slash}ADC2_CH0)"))
 (segment (start 111.39 62.29) (end 111.39 62.23) (width 1.5) (layer "F.Cu") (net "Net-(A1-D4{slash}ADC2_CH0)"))
 (segment (start 115.73 79.4) (end 111.36 79.4) (width 1.5) (layer "F.Cu") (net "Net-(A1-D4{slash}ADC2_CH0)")))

